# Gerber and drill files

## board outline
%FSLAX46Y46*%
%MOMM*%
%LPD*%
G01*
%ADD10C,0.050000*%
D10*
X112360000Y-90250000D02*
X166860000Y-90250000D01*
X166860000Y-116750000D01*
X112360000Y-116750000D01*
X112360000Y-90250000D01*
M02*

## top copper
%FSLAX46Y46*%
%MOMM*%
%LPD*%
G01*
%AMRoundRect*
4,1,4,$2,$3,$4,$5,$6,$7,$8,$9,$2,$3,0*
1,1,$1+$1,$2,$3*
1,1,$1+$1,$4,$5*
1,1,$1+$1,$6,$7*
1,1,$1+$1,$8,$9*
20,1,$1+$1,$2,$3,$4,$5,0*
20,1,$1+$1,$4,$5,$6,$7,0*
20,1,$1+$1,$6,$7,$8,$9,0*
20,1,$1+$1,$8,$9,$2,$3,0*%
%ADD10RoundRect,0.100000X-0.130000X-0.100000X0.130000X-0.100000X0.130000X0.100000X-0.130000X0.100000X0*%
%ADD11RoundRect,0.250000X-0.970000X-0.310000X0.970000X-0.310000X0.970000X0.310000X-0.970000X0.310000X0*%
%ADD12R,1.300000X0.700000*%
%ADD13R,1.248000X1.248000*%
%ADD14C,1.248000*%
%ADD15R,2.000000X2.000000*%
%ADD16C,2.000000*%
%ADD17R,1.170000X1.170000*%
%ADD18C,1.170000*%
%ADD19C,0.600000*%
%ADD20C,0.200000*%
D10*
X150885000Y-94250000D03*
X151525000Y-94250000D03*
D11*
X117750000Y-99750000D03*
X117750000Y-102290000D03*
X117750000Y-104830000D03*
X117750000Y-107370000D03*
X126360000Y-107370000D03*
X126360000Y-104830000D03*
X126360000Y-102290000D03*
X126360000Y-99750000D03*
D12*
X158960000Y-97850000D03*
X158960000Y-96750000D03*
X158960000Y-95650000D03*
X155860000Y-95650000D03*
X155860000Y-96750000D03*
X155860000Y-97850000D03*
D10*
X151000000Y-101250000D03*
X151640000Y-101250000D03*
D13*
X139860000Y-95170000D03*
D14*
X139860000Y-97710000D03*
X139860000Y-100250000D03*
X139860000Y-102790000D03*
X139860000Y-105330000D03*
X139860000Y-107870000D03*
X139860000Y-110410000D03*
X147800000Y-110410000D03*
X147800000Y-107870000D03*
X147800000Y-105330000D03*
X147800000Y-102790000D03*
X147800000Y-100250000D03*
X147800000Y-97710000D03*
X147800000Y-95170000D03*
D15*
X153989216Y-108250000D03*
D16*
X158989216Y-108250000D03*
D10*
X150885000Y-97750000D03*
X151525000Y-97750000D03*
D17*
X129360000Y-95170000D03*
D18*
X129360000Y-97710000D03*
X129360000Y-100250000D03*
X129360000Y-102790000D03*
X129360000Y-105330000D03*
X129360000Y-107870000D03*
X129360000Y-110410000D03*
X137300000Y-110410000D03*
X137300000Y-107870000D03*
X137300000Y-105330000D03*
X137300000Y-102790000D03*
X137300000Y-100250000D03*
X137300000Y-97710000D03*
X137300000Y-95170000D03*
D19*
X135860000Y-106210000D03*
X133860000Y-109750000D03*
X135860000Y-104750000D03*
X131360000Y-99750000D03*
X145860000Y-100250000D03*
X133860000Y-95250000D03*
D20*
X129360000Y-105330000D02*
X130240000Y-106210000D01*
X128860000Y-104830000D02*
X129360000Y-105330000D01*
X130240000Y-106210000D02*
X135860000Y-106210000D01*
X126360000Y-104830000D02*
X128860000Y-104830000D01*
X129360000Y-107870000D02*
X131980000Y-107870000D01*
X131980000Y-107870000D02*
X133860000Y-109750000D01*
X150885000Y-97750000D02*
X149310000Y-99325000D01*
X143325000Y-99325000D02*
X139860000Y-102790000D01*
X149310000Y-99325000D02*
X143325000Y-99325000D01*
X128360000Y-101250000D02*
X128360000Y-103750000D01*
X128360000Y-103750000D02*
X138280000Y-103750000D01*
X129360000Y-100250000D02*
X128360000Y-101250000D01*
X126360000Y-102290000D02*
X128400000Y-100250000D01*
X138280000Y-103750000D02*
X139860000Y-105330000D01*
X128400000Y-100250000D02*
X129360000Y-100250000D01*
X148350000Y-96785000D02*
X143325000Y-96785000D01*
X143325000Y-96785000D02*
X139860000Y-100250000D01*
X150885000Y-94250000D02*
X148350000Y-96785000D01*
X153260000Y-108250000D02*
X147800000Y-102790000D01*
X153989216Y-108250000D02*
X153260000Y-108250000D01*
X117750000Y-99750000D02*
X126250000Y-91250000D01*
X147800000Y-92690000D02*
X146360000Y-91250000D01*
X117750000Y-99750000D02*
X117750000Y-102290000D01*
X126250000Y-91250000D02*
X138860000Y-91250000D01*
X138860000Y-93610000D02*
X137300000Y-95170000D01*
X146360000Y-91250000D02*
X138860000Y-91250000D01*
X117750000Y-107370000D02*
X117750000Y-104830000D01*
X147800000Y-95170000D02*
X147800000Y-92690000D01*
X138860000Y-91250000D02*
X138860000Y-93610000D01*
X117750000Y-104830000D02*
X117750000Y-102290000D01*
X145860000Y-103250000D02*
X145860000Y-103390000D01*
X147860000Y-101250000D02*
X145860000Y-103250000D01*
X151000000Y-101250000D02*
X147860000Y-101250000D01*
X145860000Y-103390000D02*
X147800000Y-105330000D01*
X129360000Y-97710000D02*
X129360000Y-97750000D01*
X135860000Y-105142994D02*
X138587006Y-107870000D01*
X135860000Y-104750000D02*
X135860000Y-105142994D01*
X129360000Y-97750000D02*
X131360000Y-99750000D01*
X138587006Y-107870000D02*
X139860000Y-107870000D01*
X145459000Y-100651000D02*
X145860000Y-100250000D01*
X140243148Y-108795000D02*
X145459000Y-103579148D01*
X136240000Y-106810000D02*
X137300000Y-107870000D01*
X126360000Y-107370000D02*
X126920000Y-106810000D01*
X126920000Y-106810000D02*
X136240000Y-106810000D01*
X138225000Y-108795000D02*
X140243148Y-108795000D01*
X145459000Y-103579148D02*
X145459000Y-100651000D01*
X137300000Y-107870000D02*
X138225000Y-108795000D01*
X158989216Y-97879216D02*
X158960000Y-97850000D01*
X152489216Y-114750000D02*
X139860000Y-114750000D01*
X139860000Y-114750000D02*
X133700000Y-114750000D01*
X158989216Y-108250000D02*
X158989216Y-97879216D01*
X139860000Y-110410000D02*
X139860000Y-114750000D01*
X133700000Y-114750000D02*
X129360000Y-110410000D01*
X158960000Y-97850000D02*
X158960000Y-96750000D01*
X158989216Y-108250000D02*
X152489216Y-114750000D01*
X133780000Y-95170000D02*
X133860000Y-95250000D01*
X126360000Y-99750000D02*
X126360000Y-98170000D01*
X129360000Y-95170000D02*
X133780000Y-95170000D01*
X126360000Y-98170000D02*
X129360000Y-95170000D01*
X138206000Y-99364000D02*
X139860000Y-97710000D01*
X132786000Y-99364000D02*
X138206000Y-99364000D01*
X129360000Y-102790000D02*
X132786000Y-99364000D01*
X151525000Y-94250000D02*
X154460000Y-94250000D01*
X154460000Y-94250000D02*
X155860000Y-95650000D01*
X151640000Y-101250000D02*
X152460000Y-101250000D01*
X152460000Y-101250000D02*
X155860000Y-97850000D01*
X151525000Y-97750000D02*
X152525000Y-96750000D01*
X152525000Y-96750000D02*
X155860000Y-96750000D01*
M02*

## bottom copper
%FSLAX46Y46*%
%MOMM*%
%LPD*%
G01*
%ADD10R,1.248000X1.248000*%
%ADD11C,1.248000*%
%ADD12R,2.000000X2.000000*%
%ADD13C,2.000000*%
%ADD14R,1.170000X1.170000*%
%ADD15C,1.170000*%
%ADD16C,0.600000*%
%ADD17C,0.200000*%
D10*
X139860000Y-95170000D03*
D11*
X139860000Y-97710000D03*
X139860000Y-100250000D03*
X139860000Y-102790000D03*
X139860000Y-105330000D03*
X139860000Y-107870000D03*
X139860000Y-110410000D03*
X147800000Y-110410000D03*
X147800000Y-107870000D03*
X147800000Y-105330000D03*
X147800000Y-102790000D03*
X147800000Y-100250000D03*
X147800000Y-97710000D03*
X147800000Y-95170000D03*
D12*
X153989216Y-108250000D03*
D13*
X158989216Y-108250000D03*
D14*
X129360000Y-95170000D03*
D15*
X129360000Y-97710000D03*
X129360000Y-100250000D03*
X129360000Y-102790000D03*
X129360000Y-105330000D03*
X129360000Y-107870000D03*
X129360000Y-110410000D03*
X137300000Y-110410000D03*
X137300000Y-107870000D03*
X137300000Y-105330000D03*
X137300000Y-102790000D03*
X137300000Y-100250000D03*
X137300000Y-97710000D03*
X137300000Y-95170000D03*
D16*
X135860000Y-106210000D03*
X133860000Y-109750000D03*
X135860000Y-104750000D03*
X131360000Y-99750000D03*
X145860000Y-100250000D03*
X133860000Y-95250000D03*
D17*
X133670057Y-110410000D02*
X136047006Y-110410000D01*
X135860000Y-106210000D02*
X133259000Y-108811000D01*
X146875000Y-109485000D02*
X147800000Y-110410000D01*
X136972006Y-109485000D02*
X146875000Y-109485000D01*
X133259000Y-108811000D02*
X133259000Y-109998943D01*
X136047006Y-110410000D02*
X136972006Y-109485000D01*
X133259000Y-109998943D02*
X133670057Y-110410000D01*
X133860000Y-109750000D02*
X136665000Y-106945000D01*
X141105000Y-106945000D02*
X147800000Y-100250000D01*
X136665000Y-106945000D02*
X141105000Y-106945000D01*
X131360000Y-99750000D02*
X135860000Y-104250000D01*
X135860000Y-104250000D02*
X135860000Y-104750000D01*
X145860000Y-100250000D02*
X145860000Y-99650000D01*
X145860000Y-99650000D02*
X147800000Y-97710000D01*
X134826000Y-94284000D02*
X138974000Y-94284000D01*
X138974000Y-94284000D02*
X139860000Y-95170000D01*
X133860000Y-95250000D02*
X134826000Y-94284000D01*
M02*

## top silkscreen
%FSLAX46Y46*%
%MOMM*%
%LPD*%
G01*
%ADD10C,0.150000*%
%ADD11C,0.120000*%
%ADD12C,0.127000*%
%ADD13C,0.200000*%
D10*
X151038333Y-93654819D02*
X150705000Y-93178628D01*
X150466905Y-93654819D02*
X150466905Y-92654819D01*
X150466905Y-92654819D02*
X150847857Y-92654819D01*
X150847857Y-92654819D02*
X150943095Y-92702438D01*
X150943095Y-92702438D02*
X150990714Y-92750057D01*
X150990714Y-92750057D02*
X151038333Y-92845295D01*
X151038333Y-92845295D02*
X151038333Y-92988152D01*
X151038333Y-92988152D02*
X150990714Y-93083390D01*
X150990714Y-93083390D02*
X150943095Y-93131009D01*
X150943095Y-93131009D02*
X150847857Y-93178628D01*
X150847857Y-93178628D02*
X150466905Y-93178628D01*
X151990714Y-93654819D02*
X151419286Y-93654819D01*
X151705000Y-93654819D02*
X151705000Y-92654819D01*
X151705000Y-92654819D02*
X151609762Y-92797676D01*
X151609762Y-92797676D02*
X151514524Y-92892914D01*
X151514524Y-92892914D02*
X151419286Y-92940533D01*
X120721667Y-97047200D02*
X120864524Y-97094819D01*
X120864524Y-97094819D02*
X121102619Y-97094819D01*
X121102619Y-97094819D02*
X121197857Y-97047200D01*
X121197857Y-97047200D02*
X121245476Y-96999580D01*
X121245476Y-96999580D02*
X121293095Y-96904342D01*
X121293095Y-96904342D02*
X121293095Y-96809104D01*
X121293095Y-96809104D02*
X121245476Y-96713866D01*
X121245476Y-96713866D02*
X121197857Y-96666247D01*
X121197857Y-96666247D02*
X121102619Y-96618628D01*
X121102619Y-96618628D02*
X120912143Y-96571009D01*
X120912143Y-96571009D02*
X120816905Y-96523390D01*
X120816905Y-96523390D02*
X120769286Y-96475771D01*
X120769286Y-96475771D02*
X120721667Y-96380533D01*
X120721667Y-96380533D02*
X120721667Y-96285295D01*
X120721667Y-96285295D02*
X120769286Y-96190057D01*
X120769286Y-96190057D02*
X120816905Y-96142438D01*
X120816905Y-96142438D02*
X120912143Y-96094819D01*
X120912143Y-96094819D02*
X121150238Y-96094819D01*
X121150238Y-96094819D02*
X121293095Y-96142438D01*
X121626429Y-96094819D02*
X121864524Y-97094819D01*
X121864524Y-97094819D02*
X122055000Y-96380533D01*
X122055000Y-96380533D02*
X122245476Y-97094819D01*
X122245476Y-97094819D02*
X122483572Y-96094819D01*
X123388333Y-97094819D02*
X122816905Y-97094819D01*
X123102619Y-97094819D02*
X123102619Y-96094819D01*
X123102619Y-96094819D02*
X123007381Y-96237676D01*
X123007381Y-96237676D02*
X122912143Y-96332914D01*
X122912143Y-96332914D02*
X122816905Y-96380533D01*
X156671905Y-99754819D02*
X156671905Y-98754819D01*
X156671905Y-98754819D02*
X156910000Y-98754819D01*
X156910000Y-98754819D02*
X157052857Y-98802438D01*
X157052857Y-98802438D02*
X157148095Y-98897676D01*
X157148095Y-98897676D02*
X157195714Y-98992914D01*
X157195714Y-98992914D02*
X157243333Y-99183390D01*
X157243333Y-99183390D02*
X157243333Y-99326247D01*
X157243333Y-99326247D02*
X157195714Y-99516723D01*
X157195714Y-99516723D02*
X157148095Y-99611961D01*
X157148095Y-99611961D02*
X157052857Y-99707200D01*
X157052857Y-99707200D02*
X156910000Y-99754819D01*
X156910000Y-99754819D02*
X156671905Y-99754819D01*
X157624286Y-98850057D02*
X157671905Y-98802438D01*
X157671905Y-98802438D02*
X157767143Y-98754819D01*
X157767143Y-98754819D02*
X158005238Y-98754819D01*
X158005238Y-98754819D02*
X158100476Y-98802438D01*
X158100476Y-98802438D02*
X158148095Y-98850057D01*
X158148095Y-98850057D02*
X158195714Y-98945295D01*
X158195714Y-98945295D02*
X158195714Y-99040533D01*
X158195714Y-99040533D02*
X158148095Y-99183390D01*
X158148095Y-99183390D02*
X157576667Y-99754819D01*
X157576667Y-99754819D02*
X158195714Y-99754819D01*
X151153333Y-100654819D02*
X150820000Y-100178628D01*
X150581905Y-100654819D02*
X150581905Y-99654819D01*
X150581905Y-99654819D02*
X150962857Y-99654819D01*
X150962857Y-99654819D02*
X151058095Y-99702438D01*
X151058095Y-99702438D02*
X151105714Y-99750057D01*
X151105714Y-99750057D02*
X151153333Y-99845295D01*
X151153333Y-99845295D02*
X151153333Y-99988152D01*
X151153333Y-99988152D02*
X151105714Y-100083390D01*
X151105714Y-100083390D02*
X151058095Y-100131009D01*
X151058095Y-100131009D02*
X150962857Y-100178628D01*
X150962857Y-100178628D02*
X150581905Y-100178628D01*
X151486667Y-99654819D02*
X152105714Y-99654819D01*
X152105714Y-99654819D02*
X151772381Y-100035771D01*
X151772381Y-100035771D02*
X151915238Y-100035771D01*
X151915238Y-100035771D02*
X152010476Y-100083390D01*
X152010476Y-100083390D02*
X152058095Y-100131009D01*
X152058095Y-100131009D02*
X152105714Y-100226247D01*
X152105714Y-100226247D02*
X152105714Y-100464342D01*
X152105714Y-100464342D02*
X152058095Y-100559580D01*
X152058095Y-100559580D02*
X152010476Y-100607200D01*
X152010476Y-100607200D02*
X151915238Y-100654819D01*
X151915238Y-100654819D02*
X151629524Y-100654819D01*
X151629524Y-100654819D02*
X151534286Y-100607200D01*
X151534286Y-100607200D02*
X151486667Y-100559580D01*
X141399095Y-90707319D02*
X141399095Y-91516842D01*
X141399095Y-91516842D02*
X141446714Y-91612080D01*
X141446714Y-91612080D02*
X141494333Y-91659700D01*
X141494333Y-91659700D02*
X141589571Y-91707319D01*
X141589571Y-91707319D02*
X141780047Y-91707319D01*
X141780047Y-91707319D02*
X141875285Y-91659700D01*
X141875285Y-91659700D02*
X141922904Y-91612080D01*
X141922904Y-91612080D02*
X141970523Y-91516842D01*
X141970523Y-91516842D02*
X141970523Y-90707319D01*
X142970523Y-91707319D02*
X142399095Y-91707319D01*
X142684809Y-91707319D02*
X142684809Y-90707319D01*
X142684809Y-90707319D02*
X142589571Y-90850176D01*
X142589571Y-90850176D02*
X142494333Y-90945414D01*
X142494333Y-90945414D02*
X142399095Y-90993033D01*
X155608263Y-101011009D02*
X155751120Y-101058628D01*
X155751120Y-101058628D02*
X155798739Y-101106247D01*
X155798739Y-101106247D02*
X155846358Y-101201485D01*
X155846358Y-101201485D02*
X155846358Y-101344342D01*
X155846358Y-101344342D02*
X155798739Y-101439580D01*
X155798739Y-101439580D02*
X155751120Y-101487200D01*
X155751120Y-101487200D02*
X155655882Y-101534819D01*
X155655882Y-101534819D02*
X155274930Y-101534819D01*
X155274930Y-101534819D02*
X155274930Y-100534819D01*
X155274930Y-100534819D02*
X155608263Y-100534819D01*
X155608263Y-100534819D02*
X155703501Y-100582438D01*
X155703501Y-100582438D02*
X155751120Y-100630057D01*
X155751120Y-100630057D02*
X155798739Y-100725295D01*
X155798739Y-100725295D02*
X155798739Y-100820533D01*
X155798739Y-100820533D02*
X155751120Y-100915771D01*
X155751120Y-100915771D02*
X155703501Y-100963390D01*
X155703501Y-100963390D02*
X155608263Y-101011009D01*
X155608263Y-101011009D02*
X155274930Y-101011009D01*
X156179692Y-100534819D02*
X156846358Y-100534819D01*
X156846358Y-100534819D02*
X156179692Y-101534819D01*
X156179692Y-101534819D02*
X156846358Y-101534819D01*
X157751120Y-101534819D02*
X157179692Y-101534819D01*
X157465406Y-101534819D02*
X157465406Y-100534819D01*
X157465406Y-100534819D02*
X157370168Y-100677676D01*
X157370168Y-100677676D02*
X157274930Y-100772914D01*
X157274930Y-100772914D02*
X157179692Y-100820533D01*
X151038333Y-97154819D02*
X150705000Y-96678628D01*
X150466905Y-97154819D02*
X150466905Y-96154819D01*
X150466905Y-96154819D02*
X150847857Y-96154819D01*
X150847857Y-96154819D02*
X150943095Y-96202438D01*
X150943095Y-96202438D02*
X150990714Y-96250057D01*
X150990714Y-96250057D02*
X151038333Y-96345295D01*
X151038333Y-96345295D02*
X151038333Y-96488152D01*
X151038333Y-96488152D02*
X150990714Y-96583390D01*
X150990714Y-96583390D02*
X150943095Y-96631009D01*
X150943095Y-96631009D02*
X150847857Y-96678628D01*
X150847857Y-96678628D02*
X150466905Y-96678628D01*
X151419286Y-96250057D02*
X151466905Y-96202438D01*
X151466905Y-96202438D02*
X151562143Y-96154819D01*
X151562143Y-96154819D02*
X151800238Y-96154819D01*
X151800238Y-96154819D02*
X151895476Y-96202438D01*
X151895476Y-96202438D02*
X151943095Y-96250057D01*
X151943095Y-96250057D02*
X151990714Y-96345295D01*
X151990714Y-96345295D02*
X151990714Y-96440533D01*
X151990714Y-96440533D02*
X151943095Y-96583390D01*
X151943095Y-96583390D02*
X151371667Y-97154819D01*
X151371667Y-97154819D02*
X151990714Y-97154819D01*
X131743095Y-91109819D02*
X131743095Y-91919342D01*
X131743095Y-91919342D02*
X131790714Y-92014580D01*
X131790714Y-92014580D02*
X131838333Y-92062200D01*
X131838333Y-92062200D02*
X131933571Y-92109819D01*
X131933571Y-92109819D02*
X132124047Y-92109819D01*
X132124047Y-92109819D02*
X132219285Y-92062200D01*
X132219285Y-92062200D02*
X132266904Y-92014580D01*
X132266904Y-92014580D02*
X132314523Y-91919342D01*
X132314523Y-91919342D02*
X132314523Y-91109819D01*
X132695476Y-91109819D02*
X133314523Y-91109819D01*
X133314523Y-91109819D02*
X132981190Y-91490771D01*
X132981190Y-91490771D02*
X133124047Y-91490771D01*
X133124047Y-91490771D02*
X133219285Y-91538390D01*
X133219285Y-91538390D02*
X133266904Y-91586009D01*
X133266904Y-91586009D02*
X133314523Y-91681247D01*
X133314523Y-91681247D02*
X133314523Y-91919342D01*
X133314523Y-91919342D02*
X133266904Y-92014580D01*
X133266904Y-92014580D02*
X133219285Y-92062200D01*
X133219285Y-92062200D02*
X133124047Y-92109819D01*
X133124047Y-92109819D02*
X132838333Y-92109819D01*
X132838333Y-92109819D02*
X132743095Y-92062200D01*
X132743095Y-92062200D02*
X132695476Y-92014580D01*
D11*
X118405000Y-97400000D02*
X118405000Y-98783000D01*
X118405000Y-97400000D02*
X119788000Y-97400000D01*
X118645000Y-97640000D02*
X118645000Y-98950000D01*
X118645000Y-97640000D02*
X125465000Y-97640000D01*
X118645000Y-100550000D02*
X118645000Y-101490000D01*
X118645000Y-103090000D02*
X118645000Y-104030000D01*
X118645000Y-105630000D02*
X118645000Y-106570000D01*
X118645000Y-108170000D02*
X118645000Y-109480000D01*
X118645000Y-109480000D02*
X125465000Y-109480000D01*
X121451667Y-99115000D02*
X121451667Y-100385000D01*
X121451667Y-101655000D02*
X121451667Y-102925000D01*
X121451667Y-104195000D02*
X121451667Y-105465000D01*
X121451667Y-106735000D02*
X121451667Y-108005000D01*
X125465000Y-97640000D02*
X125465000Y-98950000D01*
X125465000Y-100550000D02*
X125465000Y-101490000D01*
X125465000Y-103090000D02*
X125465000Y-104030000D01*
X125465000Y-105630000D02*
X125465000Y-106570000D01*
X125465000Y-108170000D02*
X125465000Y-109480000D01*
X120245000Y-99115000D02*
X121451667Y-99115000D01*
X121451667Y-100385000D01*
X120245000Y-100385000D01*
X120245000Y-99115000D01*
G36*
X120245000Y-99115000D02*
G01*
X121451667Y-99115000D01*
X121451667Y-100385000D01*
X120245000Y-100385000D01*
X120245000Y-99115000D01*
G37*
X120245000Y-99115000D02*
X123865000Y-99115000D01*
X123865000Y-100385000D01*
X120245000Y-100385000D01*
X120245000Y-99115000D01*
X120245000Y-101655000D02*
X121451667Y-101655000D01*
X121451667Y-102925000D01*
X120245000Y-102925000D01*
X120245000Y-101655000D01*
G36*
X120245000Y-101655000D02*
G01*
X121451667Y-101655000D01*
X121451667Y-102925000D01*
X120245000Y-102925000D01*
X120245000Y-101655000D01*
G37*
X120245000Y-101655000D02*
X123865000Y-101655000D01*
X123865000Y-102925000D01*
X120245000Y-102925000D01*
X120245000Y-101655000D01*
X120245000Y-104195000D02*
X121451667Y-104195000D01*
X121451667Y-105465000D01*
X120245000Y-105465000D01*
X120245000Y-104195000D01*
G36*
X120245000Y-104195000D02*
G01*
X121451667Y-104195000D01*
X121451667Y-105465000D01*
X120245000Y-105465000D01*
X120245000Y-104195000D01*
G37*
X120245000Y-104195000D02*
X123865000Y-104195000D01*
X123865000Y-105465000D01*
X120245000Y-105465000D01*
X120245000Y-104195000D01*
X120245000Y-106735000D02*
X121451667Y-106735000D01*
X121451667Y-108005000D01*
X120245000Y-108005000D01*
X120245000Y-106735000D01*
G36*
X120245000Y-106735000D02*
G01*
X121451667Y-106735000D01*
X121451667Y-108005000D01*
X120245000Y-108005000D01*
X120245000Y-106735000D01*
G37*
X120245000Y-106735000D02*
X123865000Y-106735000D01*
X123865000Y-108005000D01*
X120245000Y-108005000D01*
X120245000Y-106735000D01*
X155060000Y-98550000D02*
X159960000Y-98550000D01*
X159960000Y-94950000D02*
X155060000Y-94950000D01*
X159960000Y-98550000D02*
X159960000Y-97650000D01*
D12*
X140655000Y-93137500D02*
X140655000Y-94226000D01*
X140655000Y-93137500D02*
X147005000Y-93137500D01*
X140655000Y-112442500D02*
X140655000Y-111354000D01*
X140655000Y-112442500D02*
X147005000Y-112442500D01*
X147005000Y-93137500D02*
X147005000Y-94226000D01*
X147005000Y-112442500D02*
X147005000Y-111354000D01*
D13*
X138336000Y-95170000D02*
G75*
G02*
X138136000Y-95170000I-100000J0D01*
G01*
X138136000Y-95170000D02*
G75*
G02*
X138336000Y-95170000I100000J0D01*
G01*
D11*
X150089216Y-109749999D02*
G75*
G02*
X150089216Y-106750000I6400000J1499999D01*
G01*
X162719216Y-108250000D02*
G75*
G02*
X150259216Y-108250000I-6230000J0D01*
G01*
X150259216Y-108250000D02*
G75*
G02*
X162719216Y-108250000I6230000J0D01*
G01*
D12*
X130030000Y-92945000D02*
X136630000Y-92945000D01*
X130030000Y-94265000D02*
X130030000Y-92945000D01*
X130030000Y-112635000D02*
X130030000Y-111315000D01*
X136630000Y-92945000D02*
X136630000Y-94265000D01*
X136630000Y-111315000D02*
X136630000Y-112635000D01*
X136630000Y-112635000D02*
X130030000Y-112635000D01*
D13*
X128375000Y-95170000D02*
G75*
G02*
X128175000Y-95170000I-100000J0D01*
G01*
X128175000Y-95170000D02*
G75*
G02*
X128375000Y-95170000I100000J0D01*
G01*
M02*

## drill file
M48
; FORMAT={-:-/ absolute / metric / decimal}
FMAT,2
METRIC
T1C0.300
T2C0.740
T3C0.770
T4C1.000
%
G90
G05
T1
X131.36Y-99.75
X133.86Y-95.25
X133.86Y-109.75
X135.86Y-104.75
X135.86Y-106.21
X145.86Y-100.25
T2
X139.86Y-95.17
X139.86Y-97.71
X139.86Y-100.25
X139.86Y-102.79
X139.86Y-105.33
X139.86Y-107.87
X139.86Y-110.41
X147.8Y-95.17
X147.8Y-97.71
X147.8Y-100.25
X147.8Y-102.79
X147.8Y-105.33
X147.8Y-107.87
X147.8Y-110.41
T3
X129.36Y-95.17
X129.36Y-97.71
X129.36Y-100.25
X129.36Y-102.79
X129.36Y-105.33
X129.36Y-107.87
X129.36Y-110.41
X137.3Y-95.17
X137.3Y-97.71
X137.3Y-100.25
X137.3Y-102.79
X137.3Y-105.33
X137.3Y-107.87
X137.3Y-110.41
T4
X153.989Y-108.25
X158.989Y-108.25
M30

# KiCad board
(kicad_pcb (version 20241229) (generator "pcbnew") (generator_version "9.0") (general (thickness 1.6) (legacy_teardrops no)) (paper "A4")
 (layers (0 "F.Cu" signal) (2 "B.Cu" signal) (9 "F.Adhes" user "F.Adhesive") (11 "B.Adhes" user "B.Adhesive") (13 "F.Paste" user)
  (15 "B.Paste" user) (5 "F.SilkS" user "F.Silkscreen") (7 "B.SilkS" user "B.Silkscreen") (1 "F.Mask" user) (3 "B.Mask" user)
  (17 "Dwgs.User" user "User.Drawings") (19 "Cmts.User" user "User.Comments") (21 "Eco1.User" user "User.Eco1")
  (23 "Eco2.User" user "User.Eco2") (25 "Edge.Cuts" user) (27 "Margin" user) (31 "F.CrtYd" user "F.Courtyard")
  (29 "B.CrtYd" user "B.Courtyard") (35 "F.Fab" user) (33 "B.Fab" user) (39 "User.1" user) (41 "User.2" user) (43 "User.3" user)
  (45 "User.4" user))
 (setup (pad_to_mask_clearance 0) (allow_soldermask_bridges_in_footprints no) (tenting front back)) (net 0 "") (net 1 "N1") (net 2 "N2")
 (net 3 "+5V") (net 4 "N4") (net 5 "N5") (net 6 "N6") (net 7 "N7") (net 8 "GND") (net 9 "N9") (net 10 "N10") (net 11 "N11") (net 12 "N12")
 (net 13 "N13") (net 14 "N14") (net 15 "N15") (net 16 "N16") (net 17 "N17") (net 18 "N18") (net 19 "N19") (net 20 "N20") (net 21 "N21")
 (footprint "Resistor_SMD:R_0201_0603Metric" (layer "F.Cu") (at 151.205 94.25)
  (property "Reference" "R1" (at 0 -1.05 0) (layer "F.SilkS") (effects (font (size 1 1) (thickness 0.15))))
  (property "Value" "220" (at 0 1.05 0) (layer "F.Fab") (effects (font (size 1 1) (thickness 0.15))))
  (pad "" smd roundrect (at -0.345 0) (size 0.318 0.36) (layers "F.Paste") (roundrect_rratio 0.25))
  (pad "" smd roundrect (at 0.345 0) (size 0.318 0.36) (layers "F.Paste") (roundrect_rratio 0.25))
  (pad "1" smd roundrect (at -0.32 0) (size 0.46 0.4) (layers "F.Cu" "F.Mask") (roundrect_rratio 0.25) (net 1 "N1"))
  (pad "2" smd roundrect (at 0.32 0) (size 0.46 0.4) (layers "F.Cu" "F.Mask") (roundrect_rratio 0.25) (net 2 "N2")))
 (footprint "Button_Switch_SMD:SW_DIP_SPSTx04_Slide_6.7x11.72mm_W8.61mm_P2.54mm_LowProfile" (layer "F.Cu") (at 122.055 103.56)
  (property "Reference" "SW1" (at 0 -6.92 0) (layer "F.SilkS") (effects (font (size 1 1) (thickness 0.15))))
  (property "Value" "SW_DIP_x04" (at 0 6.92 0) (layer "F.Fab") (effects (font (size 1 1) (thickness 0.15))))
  (fp_line (start -3.65 -6.16) (end -3.65 -4.777) (stroke (width 0.12) (type solid)) (layer "F.SilkS"))
  (fp_line (start -3.65 -6.16) (end -2.267 -6.16) (stroke (width 0.12) (type solid)) (layer "F.SilkS"))
  (fp_line (start -3.41 -5.92) (end -3.41 -4.61) (stroke (width 0.12) (type solid)) (layer "F.SilkS"))
  (fp_line (start -3.41 -5.92) (end 3.41 -5.92) (stroke (width 0.12) (type solid)) (layer "F.SilkS"))
  (fp_line (start -3.41 -3.01) (end -3.41 -2.07) (stroke (width 0.12) (type solid)) (layer "F.SilkS"))
  (fp_line (start -3.41 -0.47) (end -3.41 0.47) (stroke (width 0.12) (type solid)) (layer "F.SilkS"))
  (fp_line (start -3.41 2.07) (end -3.41 3.01) (stroke (width 0.12) (type solid)) (layer "F.SilkS"))
  (fp_line (start -3.41 4.61) (end -3.41 5.92) (stroke (width 0.12) (type solid)) (layer "F.SilkS"))
  (fp_line (start -3.41 5.92) (end 3.41 5.92) (stroke (width 0.12) (type solid)) (layer "F.SilkS"))
  (fp_line (start -0.603333 -4.445) (end -0.603333 -3.175) (stroke (width 0.12) (type solid)) (layer "F.SilkS"))
  (fp_line (start -0.603333 -1.905) (end -0.603333 -0.635) (stroke (width 0.12) (type solid)) (layer "F.SilkS"))
  (fp_line (start -0.603333 0.635) (end -0.603333 1.905) (stroke (width 0.12) (type solid)) (layer "F.SilkS"))
  (fp_line (start -0.603333 3.175) (end -0.603333 4.445) (stroke (width 0.12) (type solid)) (layer "F.SilkS"))
  (fp_line (start 3.41 -5.92) (end 3.41 -4.61) (stroke (width 0.12) (type solid)) (layer "F.SilkS"))
  (fp_line (start 3.41 -3.01) (end 3.41 -2.07) (stroke (width 0.12) (type solid)) (layer "F.SilkS"))
  (fp_line (start 3.41 -0.47) (end 3.41 0.47) (stroke (width 0.12) (type solid)) (layer "F.SilkS"))
  (fp_line (start 3.41 2.07) (end 3.41 3.01) (stroke (width 0.12) (type solid)) (layer "F.SilkS"))
  (fp_line (start 3.41 4.61) (end 3.41 5.92) (stroke (width 0.12) (type solid)) (layer "F.SilkS"))
  (fp_rect (start -1.81 -4.445) (end -0.603333 -3.175) (stroke (width 0.12) (type solid)) (fill yes) (layer "F.SilkS"))
  (fp_rect (start -1.81 -4.445) (end 1.81 -3.175) (stroke (width 0.12) (type solid)) (fill no) (layer "F.SilkS"))
  (fp_rect (start -1.81 -1.905) (end -0.603333 -0.635) (stroke (width 0.12) (type solid)) (fill yes) (layer "F.SilkS"))
  (fp_rect (start -1.81 -1.905) (end 1.81 -0.635) (stroke (width 0.12) (type solid)) (fill no) (layer "F.SilkS"))
  (fp_rect (start -1.81 0.635) (end -0.603333 1.905) (stroke (width 0.12) (type solid)) (fill yes) (layer "F.SilkS"))
  (fp_rect (start -1.81 0.635) (end 1.81 1.905) (stroke (width 0.12) (type solid)) (fill no) (layer "F.SilkS"))
  (fp_rect (start -1.81 3.175) (end -0.603333 4.445) (stroke (width 0.12) (type solid)) (fill yes) (layer "F.SilkS"))
  (fp_rect (start -1.81 3.175) (end 1.81 4.445) (stroke (width 0.12) (type solid)) (fill no) (layer "F.SilkS"))
  (pad "1" smd roundrect (at -4.305 -3.81) (size 2.44 1.12) (layers "F.Cu" "F.Mask" "F.Paste") (roundrect_rratio 0.223214) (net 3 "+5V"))
  (pad "2" smd roundrect (at -4.305 -1.27) (size 2.44 1.12) (layers "F.Cu" "F.Mask" "F.Paste") (roundrect_rratio 0.223214) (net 3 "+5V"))
  (pad "3" smd roundrect (at -4.305 1.27) (size 2.44 1.12) (layers "F.Cu" "F.Mask" "F.Paste") (roundrect_rratio 0.223214) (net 3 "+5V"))
  (pad "4" smd roundrect (at -4.305 3.81) (size 2.44 1.12) (layers "F.Cu" "F.Mask" "F.Paste") (roundrect_rratio 0.223214) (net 3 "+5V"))
  (pad "5" smd roundrect (at 4.305 3.81) (size 2.44 1.12) (layers "F.Cu" "F.Mask" "F.Paste") (roundrect_rratio 0.223214) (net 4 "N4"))
  (pad "6" smd roundrect (at 4.305 1.27) (size 2.44 1.12) (layers "F.Cu" "F.Mask" "F.Paste") (roundrect_rratio 0.223214) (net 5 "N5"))
  (pad "7" smd roundrect (at 4.305 -1.27) (size 2.44 1.12) (layers "F.Cu" "F.Mask" "F.Paste") (roundrect_rratio 0.223214) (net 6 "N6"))
  (pad "8" smd roundrect (at 4.305 -3.81) (size 2.44 1.12) (layers "F.Cu" "F.Mask" "F.Paste") (roundrect_rratio 0.223214) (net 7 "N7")))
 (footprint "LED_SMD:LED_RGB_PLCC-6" (layer "F.Cu") (at 157.41 96.75 180)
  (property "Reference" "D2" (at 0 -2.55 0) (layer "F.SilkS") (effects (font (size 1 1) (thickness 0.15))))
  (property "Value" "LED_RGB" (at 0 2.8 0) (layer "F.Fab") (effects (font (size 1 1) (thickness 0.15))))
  (fp_line (start 2.35 -1.8) (end -2.55 -1.8) (stroke (width 0.12) (type solid)) (layer "F.SilkS"))
  (fp_line (start -2.55 1.8) (end 2.35 1.8) (stroke (width 0.12) (type solid)) (layer "F.SilkS"))
  (fp_line (start -2.55 -1.8) (end -2.55 -0.9) (stroke (width 0.12) (type solid)) (layer "F.SilkS"))
  (pad "1" smd rect (at -1.55 -1.1 270) (size 0.7 1.3) (layers "F.Cu" "F.Mask" "F.Paste") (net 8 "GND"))
  (pad "2" smd rect (at -1.55 0 270) (size 0.7 1.3) (layers "F.Cu" "F.Mask" "F.Paste") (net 8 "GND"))
  (pad "3" smd rect (at -1.55 1.1 270) (size 0.7 1.3) (layers "F.Cu" "F.Mask" "F.Paste") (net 8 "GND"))
  (pad "4" smd rect (at 1.55 1.1 270) (size 0.7 1.3) (layers "F.Cu" "F.Mask" "F.Paste") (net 2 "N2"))
  (pad "5" smd rect (at 1.55 0 270) (size 0.7 1.3) (layers "F.Cu" "F.Mask" "F.Paste") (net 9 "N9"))
  (pad "6" smd rect (at 1.55 -1.1 270) (size 0.7 1.3) (layers "F.Cu" "F.Mask" "F.Paste") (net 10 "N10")))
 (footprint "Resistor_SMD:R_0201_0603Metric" (layer "F.Cu") (at 151.32 101.25)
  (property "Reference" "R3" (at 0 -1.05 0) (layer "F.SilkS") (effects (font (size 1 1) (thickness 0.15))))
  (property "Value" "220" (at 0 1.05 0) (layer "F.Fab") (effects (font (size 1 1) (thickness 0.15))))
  (pad "" smd roundrect (at -0.345 0) (size 0.318 0.36) (layers "F.Paste") (roundrect_rratio 0.25))
  (pad "" smd roundrect (at 0.345 0) (size 0.318 0.36) (layers "F.Paste") (roundrect_rratio 0.25))
  (pad "1" smd roundrect (at -0.32 0) (size 0.46 0.4) (layers "F.Cu" "F.Mask") (roundrect_rratio 0.25) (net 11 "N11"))
  (pad "2" smd roundrect (at 0.32 0) (size 0.46 0.4) (layers "F.Cu" "F.Mask") (roundrect_rratio 0.25) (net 10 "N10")))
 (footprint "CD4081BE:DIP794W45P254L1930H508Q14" (layer "F.Cu") (at 143.83 102.79)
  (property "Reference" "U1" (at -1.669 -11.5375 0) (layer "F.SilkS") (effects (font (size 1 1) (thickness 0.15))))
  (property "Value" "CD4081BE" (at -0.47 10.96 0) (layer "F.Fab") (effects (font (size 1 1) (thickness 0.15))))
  (fp_line (start -3.175 -9.6525) (end -3.175 -8.564) (stroke (width 0.127) (type solid)) (layer "F.SilkS"))
  (fp_line (start -3.175 -9.6525) (end 3.175 -9.6525) (stroke (width 0.127) (type solid)) (layer "F.SilkS"))
  (fp_line (start -3.175 9.6525) (end -3.175 8.564) (stroke (width 0.127) (type solid)) (layer "F.SilkS"))
  (fp_line (start -3.175 9.6525) (end 3.175 9.6525) (stroke (width 0.127) (type solid)) (layer "F.SilkS"))
  (fp_line (start 3.175 -9.6525) (end 3.175 -8.564) (stroke (width 0.127) (type solid)) (layer "F.SilkS"))
  (fp_line (start 3.175 9.6525) (end 3.175 8.564) (stroke (width 0.127) (type solid)) (layer "F.SilkS"))
  (fp_circle (center -5.594 -7.62) (end -5.494 -7.62) (stroke (width 0.2) (type solid)) (fill no) (layer "F.SilkS"))
  (pad "1" thru_hole rect (at -3.97 -7.62) (size 1.248 1.248) (drill 0.74) (layers "*.Cu" "*.Mask") (remove_unused_layers no) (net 7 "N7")
   (solder_mask_margin 0.102))
  (pad "2" thru_hole circle (at -3.97 -5.08) (size 1.248 1.248) (drill 0.74) (layers "*.Cu" "*.Mask") (remove_unused_layers no)
   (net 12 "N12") (solder_mask_margin 0.102))
  (pad "3" thru_hole circle (at -3.97 -2.54) (size 1.248 1.248) (drill 0.74) (layers "*.Cu" "*.Mask") (remove_unused_layers no) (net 1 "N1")
   (solder_mask_margin 0.102))
  (pad "4" thru_hole circle (at -3.97 0) (size 1.248 1.248) (drill 0.74) (layers "*.Cu" "*.Mask") (remove_unused_layers no) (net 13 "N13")
   (solder_mask_margin 0.102))
  (pad "5" thru_hole circle (at -3.97 2.54) (size 1.248 1.248) (drill 0.74) (layers "*.Cu" "*.Mask") (remove_unused_layers no) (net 6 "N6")
   (solder_mask_margin 0.102))
  (pad "6" thru_hole circle (at -3.97 5.08) (size 1.248 1.248) (drill 0.74) (layers "*.Cu" "*.Mask") (remove_unused_layers no)
   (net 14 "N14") (solder_mask_margin 0.102))
  (pad "7" thru_hole circle (at -3.97 7.62) (size 1.248 1.248) (drill 0.74) (layers "*.Cu" "*.Mask") (remove_unused_layers no) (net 8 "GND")
   (solder_mask_margin 0.102))
  (pad "8" thru_hole circle (at 3.97 7.62) (size 1.248 1.248) (drill 0.74) (layers "*.Cu" "*.Mask") (remove_unused_layers no) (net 5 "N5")
   (solder_mask_margin 0.102))
  (pad "9" thru_hole circle (at 3.97 5.08) (size 1.248 1.248) (drill 0.74) (layers "*.Cu" "*.Mask") (remove_unused_layers no) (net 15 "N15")
   (solder_mask_margin 0.102))
  (pad "10" thru_hole circle (at 3.97 2.54) (size 1.248 1.248) (drill 0.74) (layers "*.Cu" "*.Mask") (remove_unused_layers no)
   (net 11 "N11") (solder_mask_margin 0.102))
  (pad "11" thru_hole circle (at 3.97 0) (size 1.248 1.248) (drill 0.74) (layers "*.Cu" "*.Mask") (remove_unused_layers no) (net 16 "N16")
   (solder_mask_margin 0.102))
  (pad "12" thru_hole circle (at 3.97 -2.54) (size 1.248 1.248) (drill 0.74) (layers "*.Cu" "*.Mask") (remove_unused_layers no)
   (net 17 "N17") (solder_mask_margin 0.102))
  (pad "13" thru_hole circle (at 3.97 -5.08) (size 1.248 1.248) (drill 0.74) (layers "*.Cu" "*.Mask") (remove_unused_layers no) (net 4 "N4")
   (solder_mask_margin 0.102))
  (pad "14" thru_hole circle (at 3.97 -7.62) (size 1.248 1.248) (drill 0.74) (layers "*.Cu" "*.Mask") (remove_unused_layers no)
   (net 3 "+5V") (solder_mask_margin 0.102)))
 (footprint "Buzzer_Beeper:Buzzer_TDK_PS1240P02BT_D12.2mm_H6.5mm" (layer "F.Cu") (at 153.989216 108.25)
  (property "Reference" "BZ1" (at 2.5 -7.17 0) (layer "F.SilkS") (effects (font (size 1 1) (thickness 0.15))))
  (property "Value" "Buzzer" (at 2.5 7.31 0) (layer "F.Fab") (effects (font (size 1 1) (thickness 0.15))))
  (fp_arc (start -3.9 1.499999) (mid -4.073431 0) (end -3.9 -1.5) (stroke (width 0.12) (type solid)) (layer "F.SilkS"))
  (fp_circle (center 2.5 0) (end 8.73 0) (stroke (width 0.12) (type solid)) (fill no) (layer "F.SilkS"))
  (pad "1" thru_hole rect (at 0 0) (size 2 2) (drill 1) (layers "*.Cu" "*.Mask") (remove_unused_layers no) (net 16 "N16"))
  (pad "2" thru_hole circle (at 5 0) (size 2 2) (drill 1) (layers "*.Cu" "*.Mask") (remove_unused_layers no) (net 8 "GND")))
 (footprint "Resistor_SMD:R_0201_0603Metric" (layer "F.Cu") (at 151.205 97.75)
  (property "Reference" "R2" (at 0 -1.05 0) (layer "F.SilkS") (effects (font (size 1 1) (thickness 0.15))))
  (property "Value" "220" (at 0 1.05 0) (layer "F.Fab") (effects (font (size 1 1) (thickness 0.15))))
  (pad "" smd roundrect (at -0.345 0) (size 0.318 0.36) (layers "F.Paste") (roundrect_rratio 0.25))
  (pad "" smd roundrect (at 0.345 0) (size 0.318 0.36) (layers "F.Paste") (roundrect_rratio 0.25))
  (pad "1" smd roundrect (at -0.32 0) (size 0.46 0.4) (layers "F.Cu" "F.Mask") (roundrect_rratio 0.25) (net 13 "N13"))
  (pad "2" smd roundrect (at 0.32 0) (size 0.46 0.4) (layers "F.Cu" "F.Mask") (roundrect_rratio 0.25) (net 9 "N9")))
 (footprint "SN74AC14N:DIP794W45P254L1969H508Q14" (layer "F.Cu") (at 133.33 102.79)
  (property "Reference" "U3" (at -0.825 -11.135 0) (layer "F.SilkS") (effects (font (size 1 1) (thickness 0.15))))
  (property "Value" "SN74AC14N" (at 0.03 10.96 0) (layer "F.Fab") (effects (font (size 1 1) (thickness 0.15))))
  (fp_line (start -3.3 -9.845) (end 3.3 -9.845) (stroke (width 0.127) (type solid)) (layer "F.SilkS"))
  (fp_line (start -3.3 -8.525) (end -3.3 -9.845) (stroke (width 0.127) (type solid)) (layer "F.SilkS"))
  (fp_line (start -3.3 9.845) (end -3.3 8.525) (stroke (width 0.127) (type solid)) (layer "F.SilkS"))
  (fp_line (start 3.3 -9.845) (end 3.3 -8.525) (stroke (width 0.127) (type solid)) (layer "F.SilkS"))
  (fp_line (start 3.3 8.525) (end 3.3 9.845) (stroke (width 0.127) (type solid)) (layer "F.SilkS"))
  (fp_line (start 3.3 9.845) (end -3.3 9.845) (stroke (width 0.127) (type solid)) (layer "F.SilkS"))
  (fp_circle (center -5.055 -7.62) (end -4.955 -7.62) (stroke (width 0.2) (type solid)) (fill no) (layer "F.SilkS"))
  (pad "1" thru_hole rect (at -3.97 -7.62) (size 1.17 1.17) (drill 0.77) (layers "*.Cu" "*.Mask") (remove_unused_layers no) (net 7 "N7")
   (solder_mask_margin 0.102))
  (pad "2" thru_hole circle (at -3.97 -5.08) (size 1.17 1.17) (drill 0.77) (layers "*.Cu" "*.Mask") (remove_unused_layers no) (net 14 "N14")
   (solder_mask_margin 0.102))
  (pad "3" thru_hole circle (at -3.97 -2.54) (size 1.17 1.17) (drill 0.77) (layers "*.Cu" "*.Mask") (remove_unused_layers no) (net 6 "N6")
   (solder_mask_margin 0.102))
  (pad "4" thru_hole circle (at -3.97 0) (size 1.17 1.17) (drill 0.77) (layers "*.Cu" "*.Mask") (remove_unused_layers no) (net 12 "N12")
   (solder_mask_margin 0.102))
  (pad "5" thru_hole circle (at -3.97 2.54) (size 1.17 1.17) (drill 0.77) (layers "*.Cu" "*.Mask") (remove_unused_layers no) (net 5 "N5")
   (solder_mask_margin 0.102))
  (pad "6" thru_hole circle (at -3.97 5.08) (size 1.17 1.17) (drill 0.77) (layers "*.Cu" "*.Mask") (remove_unused_layers no) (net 17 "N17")
   (solder_mask_margin 0.102))
  (pad "7" thru_hole circle (at -3.97 7.62) (size 1.17 1.17) (drill 0.77) (layers "*.Cu" "*.Mask") (remove_unused_layers no) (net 8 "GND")
   (solder_mask_margin 0.102))
  (pad "8" thru_hole circle (at 3.97 7.62) (size 1.17 1.17) (drill 0.77) (layers "*.Cu" "*.Mask") (remove_unused_layers no) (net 15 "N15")
   (solder_mask_margin 0.102))
  (pad "9" thru_hole circle (at 3.97 5.08) (size 1.17 1.17) (drill 0.77) (layers "*.Cu" "*.Mask") (remove_unused_layers no) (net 4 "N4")
   (solder_mask_margin 0.102))
  (pad "10" thru_hole circle (at 3.97 2.54) (size 1.17 1.17) (drill 0.77) (layers "*.Cu" "*.Mask") (remove_unused_layers no) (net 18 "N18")
   (solder_mask_margin 0.102))
  (pad "11" thru_hole circle (at 3.97 0) (size 1.17 1.17) (drill 0.77) (layers "*.Cu" "*.Mask") (remove_unused_layers no) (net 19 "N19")
   (solder_mask_margin 0.102))
  (pad "12" thru_hole circle (at 3.97 -2.54) (size 1.17 1.17) (drill 0.77) (layers "*.Cu" "*.Mask") (remove_unused_layers no) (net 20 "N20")
   (solder_mask_margin 0.102))
  (pad "13" thru_hole circle (at 3.97 -5.08) (size 1.17 1.17) (drill 0.77) (layers "*.Cu" "*.Mask") (remove_unused_layers no) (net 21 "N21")
   (solder_mask_margin 0.102))
  (pad "14" thru_hole circle (at 3.97 -7.62) (size 1.17 1.17) (drill 0.77) (layers "*.Cu" "*.Mask") (remove_unused_layers no) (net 3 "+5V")
   (solder_mask_margin 0.102)))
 (gr_rect (start 112.36 90.25) (end 166.86 116.75) (stroke (width 0.05) (type default)) (fill no) (layer "Edge.Cuts"))
 (segment (start 129.36 105.33) (end 130.24 106.21) (width 0.2) (layer "F.Cu") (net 5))
 (segment (start 128.86 104.83) (end 129.36 105.33) (width 0.2) (layer "F.Cu") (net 5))
 (segment (start 130.24 106.21) (end 135.86 106.21) (width 0.2) (layer "F.Cu") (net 5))
 (segment (start 126.36 104.83) (end 128.86 104.83) (width 0.2) (layer "F.Cu") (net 5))
 (via (at 135.86 106.21) (size 0.6) (drill 0.3) (layers "F.Cu" "B.Cu") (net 5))
 (segment (start 133.670057 110.41) (end 136.047006 110.41) (width 0.2) (layer "B.Cu") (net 5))
 (segment (start 135.86 106.21) (end 133.259 108.811) (width 0.2) (layer "B.Cu") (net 5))
 (segment (start 146.875 109.485) (end 147.8 110.41) (width 0.2) (layer "B.Cu") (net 5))
 (segment (start 136.972006 109.485) (end 146.875 109.485) (width 0.2) (layer "B.Cu") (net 5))
 (segment (start 133.259 108.811) (end 133.259 109.998943) (width 0.2) (layer "B.Cu") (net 5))
 (segment (start 136.047006 110.41) (end 136.972006 109.485) (width 0.2) (layer "B.Cu") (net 5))
 (segment (start 133.259 109.998943) (end 133.670057 110.41) (width 0.2) (layer "B.Cu") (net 5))
 (segment (start 129.36 107.87) (end 131.98 107.87) (width 0.2) (layer "F.Cu") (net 17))
 (segment (start 131.98 107.87) (end 133.86 109.75) (width 0.2) (layer "F.Cu") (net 17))
 (via (at 133.86 109.75) (size 0.6) (drill 0.3) (layers "F.Cu" "B.Cu") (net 17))
 (segment (start 133.86 109.75) (end 136.665 106.945) (width 0.2) (layer "B.Cu") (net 17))
 (segment (start 141.105 106.945) (end 147.8 100.25) (width 0.2) (layer "B.Cu") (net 17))
 (segment (start 136.665 106.945) (end 141.105 106.945) (width 0.2) (layer "B.Cu") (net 17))
 (segment (start 150.885 97.75) (end 149.31 99.325) (width 0.2) (layer "F.Cu") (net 13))
 (segment (start 143.325 99.325) (end 139.86 102.79) (width 0.2) (layer "F.Cu") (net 13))
 (segment (start 149.31 99.325) (end 143.325 99.325) (width 0.2) (layer "F.Cu") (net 13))
 (segment (start 128.36 101.25) (end 128.36 103.75) (width 0.2) (layer "F.Cu") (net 6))
 (segment (start 128.36 103.75) (end 138.28 103.75) (width 0.2) (layer "F.Cu") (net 6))
 (segment (start 129.36 100.25) (end 128.36 101.25) (width 0.2) (layer "F.Cu") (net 6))
 (segment (start 126.36 102.29) (end 128.4 100.25) (width 0.2) (layer "F.Cu") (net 6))
 (segment (start 138.28 103.75) (end 139.86 105.33) (width 0.2) (layer "F.Cu") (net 6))
 (segment (start 128.4 100.25) (end 129.36 100.25) (width 0.2) (layer "F.Cu") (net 6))
 (segment (start 148.35 96.785) (end 143.325 96.785) (width 0.2) (layer "F.Cu") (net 1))
 (segment (start 143.325 96.785) (end 139.86 100.25) (width 0.2) (layer "F.Cu") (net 1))
 (segment (start 150.885 94.25) (end 148.35 96.785) (width 0.2) (layer "F.Cu") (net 1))
 (segment (start 153.26 108.25) (end 147.8 102.79) (width 0.2) (layer "F.Cu") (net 16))
 (segment (start 153.989216 108.25) (end 153.26 108.25) (width 0.2) (layer "F.Cu") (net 16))
 (segment (start 117.75 99.75) (end 126.25 91.25) (width 0.2) (layer "F.Cu") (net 3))
 (segment (start 147.8 92.69) (end 146.36 91.25) (width 0.2) (layer "F.Cu") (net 3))
 (segment (start 117.75 99.75) (end 117.75 102.29) (width 0.2) (layer "F.Cu") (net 3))
 (segment (start 126.25 91.25) (end 138.86 91.25) (width 0.2) (layer "F.Cu") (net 3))
 (segment (start 138.86 93.61) (end 137.3 95.17) (width 0.2) (layer "F.Cu") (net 3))
 (segment (start 146.36 91.25) (end 138.86 91.25) (width 0.2) (layer "F.Cu") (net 3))
 (segment (start 117.75 107.37) (end 117.75 104.83) (width 0.2) (layer "F.Cu") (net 3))
 (segment (start 147.8 95.17) (end 147.8 92.69) (width 0.2) (layer "F.Cu") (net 3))
 (segment (start 138.86 91.25) (end 138.86 93.61) (width 0.2) (layer "F.Cu") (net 3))
 (segment (start 117.75 104.83) (end 117.75 102.29) (width 0.2) (layer "F.Cu") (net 3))
 (segment (start 145.86 103.25) (end 145.86 103.39) (width 0.2) (layer "F.Cu") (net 11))
 (segment (start 147.86 101.25) (end 145.86 103.25) (width 0.2) (layer "F.Cu") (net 11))
 (segment (start 151 101.25) (end 147.86 101.25) (width 0.2) (layer "F.Cu") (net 11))
 (segment (start 145.86 103.39) (end 147.8 105.33) (width 0.2) (layer "F.Cu") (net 11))
 (segment (start 129.36 97.71) (end 129.36 97.75) (width 0.2) (layer "F.Cu") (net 14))
 (segment (start 135.86 105.142994) (end 138.587006 107.87) (width 0.2) (layer "F.Cu") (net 14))
 (segment (start 135.86 104.75) (end 135.86 105.142994) (width 0.2) (layer "F.Cu") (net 14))
 (segment (start 129.36 97.75) (end 131.36 99.75) (width 0.2) (layer "F.Cu") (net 14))
 (segment (start 138.587006 107.87) (end 139.86 107.87) (width 0.2) (layer "F.Cu") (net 14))
 (via (at 135.86 104.75) (size 0.6) (drill 0.3) (layers "F.Cu" "B.Cu") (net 14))
 (via (at 131.36 99.75) (size 0.6) (drill 0.3) (layers "F.Cu" "B.Cu") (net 14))
 (segment (start 131.36 99.75) (end 135.86 104.25) (width 0.2) (layer "B.Cu") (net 14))
 (segment (start 135.86 104.25) (end 135.86 104.75) (width 0.2) (layer "B.Cu") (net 14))
 (segment (start 145.459 100.651) (end 145.86 100.25) (width 0.2) (layer "F.Cu") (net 4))
 (segment (start 140.243148 108.795) (end 145.459 103.579148) (width 0.2) (layer "F.Cu") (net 4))
 (segment (start 136.24 106.81) (end 137.3 107.87) (width 0.2) (layer "F.Cu") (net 4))
 (segment (start 126.36 107.37) (end 126.92 106.81) (width 0.2) (layer "F.Cu") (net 4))
 (segment (start 126.92 106.81) (end 136.24 106.81) (width 0.2) (layer "F.Cu") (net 4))
 (segment (start 138.225 108.795) (end 140.243148 108.795) (width 0.2) (layer "F.Cu") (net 4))
 (segment (start 145.459 103.579148) (end 145.459 100.651) (width 0.2) (layer "F.Cu") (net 4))
 (segment (start 137.3 107.87) (end 138.225 108.795) (width 0.2) (layer "F.Cu") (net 4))
 (via (at 145.86 100.25) (size 0.6) (drill 0.3) (layers "F.Cu" "B.Cu") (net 4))
 (segment (start 145.86 100.25) (end 145.86 99.65) (width 0.2) (layer "B.Cu") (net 4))
 (segment (start 145.86 99.65) (end 147.8 97.71) (width 0.2) (layer "B.Cu") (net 4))
 (segment (start 158.989216 97.879216) (end 158.96 97.85) (width 0.2) (layer "F.Cu") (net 8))
 (segment (start 152.489216 114.75) (end 139.86 114.75) (width 0.2) (layer "F.Cu") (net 8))
 (segment (start 139.86 114.75) (end 133.7 114.75) (width 0.2) (layer "F.Cu") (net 8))
 (segment (start 158.989216 108.25) (end 158.989216 97.879216) (width 0.2) (layer "F.Cu") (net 8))
 (segment (start 139.86 110.41) (end 139.86 114.75) (width 0.2) (layer "F.Cu") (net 8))
 (segment (start 133.7 114.75) (end 129.36 110.41) (width 0.2) (layer "F.Cu") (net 8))
 (segment (start 158.96 97.85) (end 158.96 96.75) (width 0.2) (layer "F.Cu") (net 8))
 (segment (start 158.989216 108.25) (end 152.489216 114.75) (width 0.2) (layer "F.Cu") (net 8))
 (segment (start 133.78 95.17) (end 133.86 95.25) (width 0.2) (layer "F.Cu") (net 7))
 (segment (start 126.36 99.75) (end 126.36 98.17) (width 0.2) (layer "F.Cu") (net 7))
 (segment (start 129.36 95.17) (end 133.78 95.17) (width 0.2) (layer "F.Cu") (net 7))
 (segment (start 126.36 98.17) (end 129.36 95.17) (width 0.2) (layer "F.Cu") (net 7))
 (via (at 133.86 95.25) (size 0.6) (drill 0.3) (layers "F.Cu" "B.Cu") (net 7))
 (segment (start 134.826 94.284) (end 138.974 94.284) (width 0.2) (layer "B.Cu") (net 7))
 (segment (start 138.974 94.284) (end 139.86 95.17) (width 0.2) (layer "B.Cu") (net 7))
 (segment (start 133.86 95.25) (end 134.826 94.284) (width 0.2) (layer "B.Cu") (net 7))
 (segment (start 138.206 99.364) (end 139.86 97.71) (width 0.2) (layer "F.Cu") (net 12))
 (segment (start 132.786 99.364) (end 138.206 99.364) (width 0.2) (layer "F.Cu") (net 12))
 (segment (start 129.36 102.79) (end 132.786 99.364) (width 0.2) (layer "F.Cu") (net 12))
 (segment (start 151.525 94.25) (end 154.46 94.25) (width 0.2) (layer "F.Cu") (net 2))
 (segment (start 154.46 94.25) (end 155.86 95.65) (width 0.2) (layer "F.Cu") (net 2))
 (segment (start 151.64 101.25) (end 152.46 101.25) (width 0.2) (layer "F.Cu") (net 10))
 (segment (start 152.46 101.25) (end 155.86 97.85) (width 0.2) (layer "F.Cu") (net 10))
 (segment (start 151.525 97.75) (end 152.525 96.75) (width 0.2) (layer "F.Cu") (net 9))
 (segment (start 152.525 96.75) (end 155.86 96.75) (width 0.2) (layer "F.Cu") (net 9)))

